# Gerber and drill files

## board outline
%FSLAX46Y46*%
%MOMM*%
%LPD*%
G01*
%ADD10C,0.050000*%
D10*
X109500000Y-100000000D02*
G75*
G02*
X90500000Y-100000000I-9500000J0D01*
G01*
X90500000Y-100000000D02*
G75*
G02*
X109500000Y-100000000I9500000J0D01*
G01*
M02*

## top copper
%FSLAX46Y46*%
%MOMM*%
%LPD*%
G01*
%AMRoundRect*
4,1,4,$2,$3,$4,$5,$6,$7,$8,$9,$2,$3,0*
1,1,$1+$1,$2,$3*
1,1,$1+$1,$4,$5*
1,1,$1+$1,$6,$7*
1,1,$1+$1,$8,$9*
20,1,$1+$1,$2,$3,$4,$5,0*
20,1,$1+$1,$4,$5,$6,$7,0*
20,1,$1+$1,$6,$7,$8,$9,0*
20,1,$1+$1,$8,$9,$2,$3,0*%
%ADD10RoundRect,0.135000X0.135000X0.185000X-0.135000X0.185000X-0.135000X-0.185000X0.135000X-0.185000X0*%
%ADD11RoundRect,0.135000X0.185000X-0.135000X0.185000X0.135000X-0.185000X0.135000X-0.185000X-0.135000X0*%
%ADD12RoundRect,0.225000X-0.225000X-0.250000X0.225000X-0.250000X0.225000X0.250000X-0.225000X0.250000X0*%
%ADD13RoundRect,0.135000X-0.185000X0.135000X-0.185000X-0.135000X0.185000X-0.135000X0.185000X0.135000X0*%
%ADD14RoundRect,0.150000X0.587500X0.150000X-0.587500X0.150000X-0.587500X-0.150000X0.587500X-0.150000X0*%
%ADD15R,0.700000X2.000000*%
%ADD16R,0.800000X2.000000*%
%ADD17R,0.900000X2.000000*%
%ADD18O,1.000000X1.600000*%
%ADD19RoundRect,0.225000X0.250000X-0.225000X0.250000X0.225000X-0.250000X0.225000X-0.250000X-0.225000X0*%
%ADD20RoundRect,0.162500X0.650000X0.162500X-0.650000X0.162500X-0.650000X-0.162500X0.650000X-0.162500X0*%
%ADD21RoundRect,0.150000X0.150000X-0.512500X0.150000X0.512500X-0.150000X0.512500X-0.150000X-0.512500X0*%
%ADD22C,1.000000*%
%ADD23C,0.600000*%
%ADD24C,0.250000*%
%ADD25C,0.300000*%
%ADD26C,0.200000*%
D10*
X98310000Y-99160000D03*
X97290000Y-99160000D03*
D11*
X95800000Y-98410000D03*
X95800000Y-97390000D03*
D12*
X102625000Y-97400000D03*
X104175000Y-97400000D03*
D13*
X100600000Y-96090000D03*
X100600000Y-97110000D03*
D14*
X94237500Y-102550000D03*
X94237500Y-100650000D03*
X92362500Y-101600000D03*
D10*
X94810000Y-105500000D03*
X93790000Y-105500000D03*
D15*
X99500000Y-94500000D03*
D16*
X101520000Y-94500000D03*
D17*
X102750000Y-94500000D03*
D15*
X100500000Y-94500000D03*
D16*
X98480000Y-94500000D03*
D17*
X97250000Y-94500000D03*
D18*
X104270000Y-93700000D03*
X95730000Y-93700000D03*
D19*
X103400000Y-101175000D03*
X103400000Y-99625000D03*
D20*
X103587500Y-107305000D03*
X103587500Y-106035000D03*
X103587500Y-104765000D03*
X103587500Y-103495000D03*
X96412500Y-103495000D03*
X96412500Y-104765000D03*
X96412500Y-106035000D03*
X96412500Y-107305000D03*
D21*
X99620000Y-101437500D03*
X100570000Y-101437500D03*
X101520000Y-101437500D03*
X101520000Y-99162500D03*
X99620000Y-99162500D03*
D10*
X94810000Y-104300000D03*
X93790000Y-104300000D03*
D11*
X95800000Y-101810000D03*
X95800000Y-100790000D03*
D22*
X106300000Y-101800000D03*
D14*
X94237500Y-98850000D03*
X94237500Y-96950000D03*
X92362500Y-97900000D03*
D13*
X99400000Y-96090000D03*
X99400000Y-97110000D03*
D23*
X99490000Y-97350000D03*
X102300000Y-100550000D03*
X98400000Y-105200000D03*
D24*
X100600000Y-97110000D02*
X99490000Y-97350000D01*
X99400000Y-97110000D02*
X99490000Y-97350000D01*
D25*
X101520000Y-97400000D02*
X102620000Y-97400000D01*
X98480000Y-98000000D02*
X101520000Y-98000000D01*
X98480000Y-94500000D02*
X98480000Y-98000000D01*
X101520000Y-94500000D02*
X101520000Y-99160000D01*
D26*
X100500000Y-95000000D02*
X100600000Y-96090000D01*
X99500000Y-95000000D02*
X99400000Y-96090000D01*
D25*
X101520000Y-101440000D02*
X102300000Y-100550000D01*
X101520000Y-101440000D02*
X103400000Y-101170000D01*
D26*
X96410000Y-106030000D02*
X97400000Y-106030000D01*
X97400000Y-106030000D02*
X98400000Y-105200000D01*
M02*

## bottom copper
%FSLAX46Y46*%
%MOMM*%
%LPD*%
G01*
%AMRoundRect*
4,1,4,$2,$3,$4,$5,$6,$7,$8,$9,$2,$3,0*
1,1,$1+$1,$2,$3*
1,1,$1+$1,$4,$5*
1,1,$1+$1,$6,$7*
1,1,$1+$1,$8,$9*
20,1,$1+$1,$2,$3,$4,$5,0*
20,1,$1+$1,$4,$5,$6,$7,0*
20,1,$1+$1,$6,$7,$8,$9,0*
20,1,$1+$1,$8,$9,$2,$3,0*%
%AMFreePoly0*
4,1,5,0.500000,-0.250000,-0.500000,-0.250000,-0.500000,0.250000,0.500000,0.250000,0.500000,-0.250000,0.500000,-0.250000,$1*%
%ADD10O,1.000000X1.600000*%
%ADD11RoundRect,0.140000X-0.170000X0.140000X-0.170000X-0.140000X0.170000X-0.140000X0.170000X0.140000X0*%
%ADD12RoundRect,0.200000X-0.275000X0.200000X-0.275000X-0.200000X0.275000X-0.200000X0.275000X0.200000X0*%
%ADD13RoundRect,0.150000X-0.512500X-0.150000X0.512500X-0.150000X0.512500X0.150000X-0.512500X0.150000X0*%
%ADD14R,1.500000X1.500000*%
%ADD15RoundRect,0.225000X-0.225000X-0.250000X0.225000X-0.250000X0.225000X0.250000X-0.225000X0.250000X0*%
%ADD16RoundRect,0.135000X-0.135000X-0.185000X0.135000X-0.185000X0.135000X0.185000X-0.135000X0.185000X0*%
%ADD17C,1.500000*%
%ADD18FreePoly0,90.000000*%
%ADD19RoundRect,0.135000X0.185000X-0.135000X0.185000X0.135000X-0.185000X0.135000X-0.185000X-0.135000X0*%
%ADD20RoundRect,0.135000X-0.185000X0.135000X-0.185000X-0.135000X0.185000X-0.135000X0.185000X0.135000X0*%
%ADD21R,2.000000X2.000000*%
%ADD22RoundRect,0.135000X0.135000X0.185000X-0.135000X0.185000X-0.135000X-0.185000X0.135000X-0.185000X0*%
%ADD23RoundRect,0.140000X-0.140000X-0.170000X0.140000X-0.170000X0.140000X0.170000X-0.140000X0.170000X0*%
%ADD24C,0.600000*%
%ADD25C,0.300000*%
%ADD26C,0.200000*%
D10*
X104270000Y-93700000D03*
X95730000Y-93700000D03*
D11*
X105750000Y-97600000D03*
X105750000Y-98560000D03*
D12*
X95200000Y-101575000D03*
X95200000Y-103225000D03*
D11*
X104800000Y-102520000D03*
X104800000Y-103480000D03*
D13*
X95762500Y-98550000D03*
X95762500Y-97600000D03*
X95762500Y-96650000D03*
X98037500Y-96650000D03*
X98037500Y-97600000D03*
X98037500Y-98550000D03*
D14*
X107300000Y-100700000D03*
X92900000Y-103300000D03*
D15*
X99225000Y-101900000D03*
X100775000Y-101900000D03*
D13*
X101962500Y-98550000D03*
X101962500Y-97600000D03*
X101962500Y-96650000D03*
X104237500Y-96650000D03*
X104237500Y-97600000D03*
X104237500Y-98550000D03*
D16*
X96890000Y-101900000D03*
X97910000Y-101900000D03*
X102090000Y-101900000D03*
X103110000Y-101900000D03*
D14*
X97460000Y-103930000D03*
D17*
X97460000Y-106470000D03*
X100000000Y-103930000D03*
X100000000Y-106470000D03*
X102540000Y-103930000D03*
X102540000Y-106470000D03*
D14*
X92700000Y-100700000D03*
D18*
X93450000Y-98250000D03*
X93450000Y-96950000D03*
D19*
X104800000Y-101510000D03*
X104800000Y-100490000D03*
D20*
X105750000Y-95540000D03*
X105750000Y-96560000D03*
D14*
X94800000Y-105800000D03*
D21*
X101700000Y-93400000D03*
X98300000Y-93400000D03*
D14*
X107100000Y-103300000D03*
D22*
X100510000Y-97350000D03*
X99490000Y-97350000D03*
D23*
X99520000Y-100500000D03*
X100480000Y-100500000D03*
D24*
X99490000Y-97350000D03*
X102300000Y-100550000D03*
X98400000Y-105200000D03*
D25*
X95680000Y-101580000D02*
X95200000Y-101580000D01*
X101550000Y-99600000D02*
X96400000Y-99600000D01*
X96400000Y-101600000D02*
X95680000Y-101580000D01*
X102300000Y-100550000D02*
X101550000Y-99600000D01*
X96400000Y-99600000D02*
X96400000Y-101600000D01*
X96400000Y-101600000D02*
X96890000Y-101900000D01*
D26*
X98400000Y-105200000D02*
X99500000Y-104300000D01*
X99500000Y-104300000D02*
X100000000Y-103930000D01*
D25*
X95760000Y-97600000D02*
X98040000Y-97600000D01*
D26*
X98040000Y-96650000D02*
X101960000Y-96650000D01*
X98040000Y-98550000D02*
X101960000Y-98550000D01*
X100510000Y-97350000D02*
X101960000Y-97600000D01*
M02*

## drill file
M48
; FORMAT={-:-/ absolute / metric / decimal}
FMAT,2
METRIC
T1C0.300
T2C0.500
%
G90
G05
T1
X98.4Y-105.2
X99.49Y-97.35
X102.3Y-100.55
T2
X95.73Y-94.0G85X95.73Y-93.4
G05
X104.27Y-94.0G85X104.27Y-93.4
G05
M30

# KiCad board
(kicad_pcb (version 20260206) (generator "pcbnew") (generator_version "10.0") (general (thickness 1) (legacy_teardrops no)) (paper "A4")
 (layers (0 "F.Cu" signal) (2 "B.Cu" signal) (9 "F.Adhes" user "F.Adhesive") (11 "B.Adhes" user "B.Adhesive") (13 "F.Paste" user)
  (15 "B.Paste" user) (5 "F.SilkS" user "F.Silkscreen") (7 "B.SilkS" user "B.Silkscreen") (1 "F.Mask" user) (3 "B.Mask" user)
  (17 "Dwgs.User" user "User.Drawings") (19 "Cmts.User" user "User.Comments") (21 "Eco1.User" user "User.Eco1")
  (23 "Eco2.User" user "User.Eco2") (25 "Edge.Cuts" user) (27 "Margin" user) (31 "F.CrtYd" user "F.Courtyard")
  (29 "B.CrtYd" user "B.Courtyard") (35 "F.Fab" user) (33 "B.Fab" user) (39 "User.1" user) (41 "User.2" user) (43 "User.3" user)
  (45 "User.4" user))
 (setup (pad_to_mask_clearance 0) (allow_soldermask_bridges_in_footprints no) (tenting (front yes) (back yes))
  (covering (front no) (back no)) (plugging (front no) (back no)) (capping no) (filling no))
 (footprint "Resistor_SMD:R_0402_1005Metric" (layer "F.Cu") (at 97.8 99.16 180)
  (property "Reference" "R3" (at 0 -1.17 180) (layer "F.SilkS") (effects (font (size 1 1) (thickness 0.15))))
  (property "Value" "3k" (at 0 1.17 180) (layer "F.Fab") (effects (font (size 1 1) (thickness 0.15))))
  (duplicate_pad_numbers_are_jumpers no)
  (pad "1" smd roundrect (at -0.51 0 180) (size 0.54 0.64) (layers "F.Cu" "F.Mask" "F.Paste") (roundrect_rratio 0.25) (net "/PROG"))
  (pad "2" smd roundrect (at 0.51 0 180) (size 0.54 0.64) (layers "F.Cu" "F.Mask" "F.Paste") (roundrect_rratio 0.25) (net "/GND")))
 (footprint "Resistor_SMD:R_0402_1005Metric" (layer "F.Cu") (at 95.8 97.9 90)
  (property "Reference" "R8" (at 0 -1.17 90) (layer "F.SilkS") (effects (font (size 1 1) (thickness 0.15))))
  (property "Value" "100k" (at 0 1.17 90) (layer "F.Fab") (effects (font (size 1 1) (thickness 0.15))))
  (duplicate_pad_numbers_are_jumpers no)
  (pad "1" smd roundrect (at -0.51 0 90) (size 0.54 0.64) (layers "F.Cu" "F.Mask" "F.Paste") (roundrect_rratio 0.25) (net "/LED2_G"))
  (pad "2" smd roundrect (at 0.51 0 90) (size 0.54 0.64) (layers "F.Cu" "F.Mask" "F.Paste") (roundrect_rratio 0.25) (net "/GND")))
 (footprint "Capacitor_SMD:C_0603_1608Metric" (layer "F.Cu") (at 103.4 97.4)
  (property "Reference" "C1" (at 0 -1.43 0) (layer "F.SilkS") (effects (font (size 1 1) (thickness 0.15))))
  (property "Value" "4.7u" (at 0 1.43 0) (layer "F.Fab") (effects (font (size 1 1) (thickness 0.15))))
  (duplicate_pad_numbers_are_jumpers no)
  (pad "1" smd roundrect (at -0.775 0) (size 0.9 0.95) (layers "F.Cu" "F.Mask" "F.Paste") (roundrect_rratio 0.25) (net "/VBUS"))
  (pad "2" smd roundrect (at 0.775 0) (size 0.9 0.95) (layers "F.Cu" "F.Mask" "F.Paste") (roundrect_rratio 0.25) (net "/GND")))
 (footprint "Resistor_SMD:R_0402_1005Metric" (layer "F.Cu") (at 100.6 96.6 -90)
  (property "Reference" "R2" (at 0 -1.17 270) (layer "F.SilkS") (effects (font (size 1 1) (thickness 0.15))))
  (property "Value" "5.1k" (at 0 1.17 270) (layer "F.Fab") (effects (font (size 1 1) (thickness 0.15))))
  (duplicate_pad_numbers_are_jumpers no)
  (pad "1" smd roundrect (at -0.51 0 270) (size 0.54 0.64) (layers "F.Cu" "F.Mask" "F.Paste") (roundrect_rratio 0.25) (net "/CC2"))
  (pad "2" smd roundrect (at 0.51 0 270) (size 0.54 0.64) (layers "F.Cu" "F.Mask" "F.Paste") (roundrect_rratio 0.25) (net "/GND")))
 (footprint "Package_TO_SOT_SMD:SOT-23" (layer "F.Cu") (at 93.3 101.6 180)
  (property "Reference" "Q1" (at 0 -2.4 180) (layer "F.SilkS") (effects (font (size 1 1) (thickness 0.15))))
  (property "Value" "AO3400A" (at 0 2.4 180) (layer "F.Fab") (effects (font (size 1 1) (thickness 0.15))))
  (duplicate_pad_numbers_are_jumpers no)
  (pad "1" smd roundrect (at -0.9375 -0.95 180) (size 1.475 0.6) (layers "F.Cu" "F.Mask" "F.Paste") (roundrect_rratio 0.25) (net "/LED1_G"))
  (pad "2" smd roundrect (at -0.9375 0.95 180) (size 1.475 0.6) (layers "F.Cu" "F.Mask" "F.Paste") (roundrect_rratio 0.25) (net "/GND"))
  (pad "3" smd roundrect (at 0.9375 0 180) (size 1.475 0.6) (layers "F.Cu" "F.Mask" "F.Paste") (roundrect_rratio 0.25) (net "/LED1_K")))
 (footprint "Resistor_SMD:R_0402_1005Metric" (layer "F.Cu") (at 94.3 105.5 180)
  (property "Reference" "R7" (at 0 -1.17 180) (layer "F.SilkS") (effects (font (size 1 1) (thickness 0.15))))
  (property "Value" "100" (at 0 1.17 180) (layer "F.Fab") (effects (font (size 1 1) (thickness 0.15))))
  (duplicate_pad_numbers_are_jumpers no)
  (pad "1" smd roundrect (at -0.51 0 180) (size 0.54 0.64) (layers "F.Cu" "F.Mask" "F.Paste") (roundrect_rratio 0.25) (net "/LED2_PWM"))
  (pad "2" smd roundrect (at 0.51 0 180) (size 0.54 0.64) (layers "F.Cu" "F.Mask" "F.Paste") (roundrect_rratio 0.25) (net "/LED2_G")))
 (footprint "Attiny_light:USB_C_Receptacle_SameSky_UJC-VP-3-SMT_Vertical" (layer "F.Cu") (at 100 94.5 180)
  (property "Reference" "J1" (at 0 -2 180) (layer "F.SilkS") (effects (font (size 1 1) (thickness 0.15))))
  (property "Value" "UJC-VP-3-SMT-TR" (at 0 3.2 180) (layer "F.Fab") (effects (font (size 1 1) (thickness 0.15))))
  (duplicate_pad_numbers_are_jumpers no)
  (pad "A5" smd rect (at 0.5 0 180) (size 0.7 2) (layers "F.Cu" "F.Mask" "F.Paste") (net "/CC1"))
  (pad "A9" smd rect (at -1.52 0 180) (size 0.8 2) (layers "F.Cu" "F.Mask" "F.Paste") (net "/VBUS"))
  (pad "A12" smd rect (at -2.75 0 180) (size 0.9 2) (layers "F.Cu" "F.Mask" "F.Paste") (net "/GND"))
  (pad "B5" smd rect (at -0.5 0 180) (size 0.7 2) (layers "F.Cu" "F.Mask" "F.Paste") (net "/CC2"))
  (pad "B9" smd rect (at 1.52 0 180) (size 0.8 2) (layers "F.Cu" "F.Mask" "F.Paste") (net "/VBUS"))
  (pad "B12" smd rect (at 2.75 0 180) (size 0.9 2) (layers "F.Cu" "F.Mask" "F.Paste") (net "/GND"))
  (pad "SH" thru_hole oval (at -4.27 0.8 180) (size 1 1.6) (drill oval 0.5 1.1) (layers "*.Cu" "*.Mask") (remove_unused_layers no)
   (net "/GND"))
  (pad "SH" thru_hole oval (at 4.27 0.8 180) (size 1 1.6) (drill oval 0.5 1.1) (layers "*.Cu" "*.Mask") (remove_unused_layers no)
   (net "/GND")))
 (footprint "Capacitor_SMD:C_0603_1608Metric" (layer "F.Cu") (at 103.4 100.4 90)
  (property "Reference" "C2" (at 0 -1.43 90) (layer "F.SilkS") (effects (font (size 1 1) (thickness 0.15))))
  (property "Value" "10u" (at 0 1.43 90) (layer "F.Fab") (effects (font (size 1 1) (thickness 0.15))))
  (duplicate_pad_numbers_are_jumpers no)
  (pad "1" smd roundrect (at -0.775 0 90) (size 0.9 0.95) (layers "F.Cu" "F.Mask" "F.Paste") (roundrect_rratio 0.25) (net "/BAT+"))
  (pad "2" smd roundrect (at 0.775 0 90) (size 0.9 0.95) (layers "F.Cu" "F.Mask" "F.Paste") (roundrect_rratio 0.25) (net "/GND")))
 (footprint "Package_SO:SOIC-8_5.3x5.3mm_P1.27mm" (layer "F.Cu") (at 100 105.4 180)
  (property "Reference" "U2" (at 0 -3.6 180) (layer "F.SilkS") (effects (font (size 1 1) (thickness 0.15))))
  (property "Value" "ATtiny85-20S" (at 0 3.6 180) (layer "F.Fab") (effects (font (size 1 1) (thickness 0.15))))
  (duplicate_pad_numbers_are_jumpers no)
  (pad "1" smd roundrect (at -3.5875 -1.905 180) (size 1.625 0.65) (layers "F.Cu" "F.Mask" "F.Paste") (roundrect_rratio 0.25) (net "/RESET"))
  (pad "2" smd roundrect (at -3.5875 -0.635 180) (size 1.625 0.65) (layers "F.Cu" "F.Mask" "F.Paste") (roundrect_rratio 0.25) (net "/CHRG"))
  (pad "3" smd roundrect (at -3.5875 0.635 180) (size 1.625 0.65) (layers "F.Cu" "F.Mask" "F.Paste") (roundrect_rratio 0.25) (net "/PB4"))
  (pad "4" smd roundrect (at -3.5875 1.905 180) (size 1.625 0.65) (layers "F.Cu" "F.Mask" "F.Paste") (roundrect_rratio 0.25) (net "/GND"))
  (pad "5" smd roundrect (at 3.5875 1.905 180) (size 1.625 0.65) (layers "F.Cu" "F.Mask" "F.Paste") (roundrect_rratio 0.25)
   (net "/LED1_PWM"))
  (pad "6" smd roundrect (at 3.5875 0.635 180) (size 1.625 0.65) (layers "F.Cu" "F.Mask" "F.Paste") (roundrect_rratio 0.25)
   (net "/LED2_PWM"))
  (pad "7" smd roundrect (at 3.5875 -0.635 180) (size 1.625 0.65) (layers "F.Cu" "F.Mask" "F.Paste") (roundrect_rratio 0.25) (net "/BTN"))
  (pad "8" smd roundrect (at 3.5875 -1.905 180) (size 1.625 0.65) (layers "F.Cu" "F.Mask" "F.Paste") (roundrect_rratio 0.25) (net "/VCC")))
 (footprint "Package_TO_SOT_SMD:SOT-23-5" (layer "F.Cu") (at 100.57 100.3 90)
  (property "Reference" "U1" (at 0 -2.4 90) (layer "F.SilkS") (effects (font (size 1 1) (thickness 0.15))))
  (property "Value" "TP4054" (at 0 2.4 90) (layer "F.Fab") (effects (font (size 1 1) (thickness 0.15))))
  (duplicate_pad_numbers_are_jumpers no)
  (pad "1" smd roundrect (at -1.1375 -0.95 90) (size 1.325 0.6) (layers "F.Cu" "F.Mask" "F.Paste") (roundrect_rratio 0.25) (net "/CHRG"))
  (pad "2" smd roundrect (at -1.1375 0 90) (size 1.325 0.6) (layers "F.Cu" "F.Mask" "F.Paste") (roundrect_rratio 0.25) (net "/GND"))
  (pad "3" smd roundrect (at -1.1375 0.95 90) (size 1.325 0.6) (layers "F.Cu" "F.Mask" "F.Paste") (roundrect_rratio 0.25) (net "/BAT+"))
  (pad "4" smd roundrect (at 1.1375 0.95 90) (size 1.325 0.6) (layers "F.Cu" "F.Mask" "F.Paste") (roundrect_rratio 0.25) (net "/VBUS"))
  (pad "5" smd roundrect (at 1.1375 -0.95 90) (size 1.325 0.6) (layers "F.Cu" "F.Mask" "F.Paste") (roundrect_rratio 0.25) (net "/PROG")))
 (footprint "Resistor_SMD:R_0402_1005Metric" (layer "F.Cu") (at 94.3 104.3 180)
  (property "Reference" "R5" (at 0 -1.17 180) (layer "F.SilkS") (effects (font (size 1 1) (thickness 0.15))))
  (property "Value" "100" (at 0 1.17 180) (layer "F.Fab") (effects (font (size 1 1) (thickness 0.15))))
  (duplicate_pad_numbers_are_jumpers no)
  (pad "1" smd roundrect (at -0.51 0 180) (size 0.54 0.64) (layers "F.Cu" "F.Mask" "F.Paste") (roundrect_rratio 0.25) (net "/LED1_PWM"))
  (pad "2" smd roundrect (at 0.51 0 180) (size 0.54 0.64) (layers "F.Cu" "F.Mask" "F.Paste") (roundrect_rratio 0.25) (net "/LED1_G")))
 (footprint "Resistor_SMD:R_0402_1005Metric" (layer "F.Cu") (at 95.8 101.3 90)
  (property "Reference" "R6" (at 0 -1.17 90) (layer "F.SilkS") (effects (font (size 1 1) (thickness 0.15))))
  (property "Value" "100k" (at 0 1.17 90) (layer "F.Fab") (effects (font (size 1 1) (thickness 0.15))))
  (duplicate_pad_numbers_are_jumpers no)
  (pad "1" smd roundrect (at -0.51 0 90) (size 0.54 0.64) (layers "F.Cu" "F.Mask" "F.Paste") (roundrect_rratio 0.25) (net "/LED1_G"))
  (pad "2" smd roundrect (at 0.51 0 90) (size 0.54 0.64) (layers "F.Cu" "F.Mask" "F.Paste") (roundrect_rratio 0.25) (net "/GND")))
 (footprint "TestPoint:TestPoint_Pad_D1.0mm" (layer "F.Cu") (at 106.3 101.8)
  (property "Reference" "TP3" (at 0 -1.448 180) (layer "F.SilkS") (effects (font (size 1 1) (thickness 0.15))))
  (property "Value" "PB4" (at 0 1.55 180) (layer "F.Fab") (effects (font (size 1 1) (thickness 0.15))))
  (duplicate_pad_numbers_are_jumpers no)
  (pad "1" smd circle (at 0 0) (size 1 1) (layers "F.Cu" "F.Mask") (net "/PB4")))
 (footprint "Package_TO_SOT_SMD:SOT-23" (layer "F.Cu") (at 93.3 97.9 180)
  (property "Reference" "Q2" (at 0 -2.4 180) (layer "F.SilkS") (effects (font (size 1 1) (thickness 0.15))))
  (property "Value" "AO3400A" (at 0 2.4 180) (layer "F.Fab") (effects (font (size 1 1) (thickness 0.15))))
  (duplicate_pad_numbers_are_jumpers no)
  (pad "1" smd roundrect (at -0.9375 -0.95 180) (size 1.475 0.6) (layers "F.Cu" "F.Mask" "F.Paste") (roundrect_rratio 0.25) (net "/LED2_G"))
  (pad "2" smd roundrect (at -0.9375 0.95 180) (size 1.475 0.6) (layers "F.Cu" "F.Mask" "F.Paste") (roundrect_rratio 0.25) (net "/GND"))
  (pad "3" smd roundrect (at 0.9375 0 180) (size 1.475 0.6) (layers "F.Cu" "F.Mask" "F.Paste") (roundrect_rratio 0.25) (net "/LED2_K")))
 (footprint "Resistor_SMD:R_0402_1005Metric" (layer "F.Cu") (at 99.4 96.6 -90)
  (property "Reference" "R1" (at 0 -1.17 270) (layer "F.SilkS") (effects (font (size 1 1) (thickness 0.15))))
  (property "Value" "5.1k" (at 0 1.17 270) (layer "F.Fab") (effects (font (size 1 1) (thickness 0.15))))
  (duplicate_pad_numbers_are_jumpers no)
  (pad "1" smd roundrect (at -0.51 0 270) (size 0.54 0.64) (layers "F.Cu" "F.Mask" "F.Paste") (roundrect_rratio 0.25) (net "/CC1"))
  (pad "2" smd roundrect (at 0.51 0 270) (size 0.54 0.64) (layers "F.Cu" "F.Mask" "F.Paste") (roundrect_rratio 0.25) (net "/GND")))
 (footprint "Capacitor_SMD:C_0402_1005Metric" (layer "B.Cu") (at 105.75 98.08 -90)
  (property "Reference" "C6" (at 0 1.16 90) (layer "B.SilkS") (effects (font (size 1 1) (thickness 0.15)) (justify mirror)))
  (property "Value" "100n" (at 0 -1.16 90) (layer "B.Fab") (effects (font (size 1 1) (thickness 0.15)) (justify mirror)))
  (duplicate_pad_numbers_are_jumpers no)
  (pad "1" smd roundrect (at -0.48 0 270) (size 0.56 0.62) (layers "B.Cu" "B.Mask" "B.Paste") (roundrect_rratio 0.25) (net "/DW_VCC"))
  (pad "2" smd roundrect (at 0.48 0 270) (size 0.56 0.62) (layers "B.Cu" "B.Mask" "B.Paste") (roundrect_rratio 0.25) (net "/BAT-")))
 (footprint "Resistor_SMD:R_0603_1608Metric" (layer "B.Cu") (at 95.2 102.4 -90)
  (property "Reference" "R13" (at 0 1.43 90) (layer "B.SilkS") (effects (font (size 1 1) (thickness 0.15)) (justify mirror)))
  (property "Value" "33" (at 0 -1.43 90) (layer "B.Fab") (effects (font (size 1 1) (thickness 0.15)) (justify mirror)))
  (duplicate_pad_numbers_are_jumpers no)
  (pad "1" smd roundrect (at -0.825 0 270) (size 0.8 0.95) (layers "B.Cu" "B.Mask" "B.Paste") (roundrect_rratio 0.25) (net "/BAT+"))
  (pad "2" smd roundrect (at 0.825 0 270) (size 0.8 0.95) (layers "B.Cu" "B.Mask" "B.Paste") (roundrect_rratio 0.25) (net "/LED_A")))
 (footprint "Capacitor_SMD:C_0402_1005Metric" (layer "B.Cu") (at 104.8 103 -90)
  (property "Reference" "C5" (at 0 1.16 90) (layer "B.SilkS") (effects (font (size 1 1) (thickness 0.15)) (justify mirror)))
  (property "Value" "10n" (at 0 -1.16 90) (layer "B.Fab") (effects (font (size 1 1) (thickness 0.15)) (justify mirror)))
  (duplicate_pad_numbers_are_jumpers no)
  (pad "1" smd roundrect (at -0.48 0 270) (size 0.56 0.62) (layers "B.Cu" "B.Mask" "B.Paste") (roundrect_rratio 0.25) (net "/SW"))
  (pad "2" smd roundrect (at 0.48 0 270) (size 0.56 0.62) (layers "B.Cu" "B.Mask" "B.Paste") (roundrect_rratio 0.25) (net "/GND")))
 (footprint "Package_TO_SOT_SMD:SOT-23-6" (layer "B.Cu") (at 96.9 97.6)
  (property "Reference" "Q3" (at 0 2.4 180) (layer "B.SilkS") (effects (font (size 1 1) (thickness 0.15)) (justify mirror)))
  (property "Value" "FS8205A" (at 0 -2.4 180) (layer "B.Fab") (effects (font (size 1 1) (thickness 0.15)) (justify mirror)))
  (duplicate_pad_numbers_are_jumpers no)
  (pad "1" smd roundrect (at -1.1375 0.95) (size 1.325 0.6) (layers "B.Cu" "B.Mask" "B.Paste") (roundrect_rratio 0.25) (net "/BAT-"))
  (pad "2" smd roundrect (at -1.1375 0) (size 1.325 0.6) (layers "B.Cu" "B.Mask" "B.Paste") (roundrect_rratio 0.25) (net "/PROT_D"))
  (pad "3" smd roundrect (at -1.1375 -0.95) (size 1.325 0.6) (layers "B.Cu" "B.Mask" "B.Paste") (roundrect_rratio 0.25) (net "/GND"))
  (pad "4" smd roundrect (at 1.1375 -0.95) (size 1.325 0.6) (layers "B.Cu" "B.Mask" "B.Paste") (roundrect_rratio 0.25) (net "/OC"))
  (pad "5" smd roundrect (at 1.1375 0) (size 1.325 0.6) (layers "B.Cu" "B.Mask" "B.Paste") (roundrect_rratio 0.25) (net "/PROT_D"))
  (pad "6" smd roundrect (at 1.1375 0.95) (size 1.325 0.6) (layers "B.Cu" "B.Mask" "B.Paste") (roundrect_rratio 0.25) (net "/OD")))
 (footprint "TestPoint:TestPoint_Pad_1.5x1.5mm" (layer "B.Cu") (at 107.3 100.7)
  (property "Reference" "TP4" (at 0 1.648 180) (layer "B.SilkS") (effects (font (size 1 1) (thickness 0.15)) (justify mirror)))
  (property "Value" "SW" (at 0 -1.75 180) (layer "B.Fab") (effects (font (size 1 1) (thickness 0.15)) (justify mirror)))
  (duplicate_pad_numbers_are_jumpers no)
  (pad "1" smd rect (at 0 0) (size 1.5 1.5) (layers "B.Cu" "B.Mask") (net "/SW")))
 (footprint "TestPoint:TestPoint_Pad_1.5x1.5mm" (layer "B.Cu") (at 92.9 103.3)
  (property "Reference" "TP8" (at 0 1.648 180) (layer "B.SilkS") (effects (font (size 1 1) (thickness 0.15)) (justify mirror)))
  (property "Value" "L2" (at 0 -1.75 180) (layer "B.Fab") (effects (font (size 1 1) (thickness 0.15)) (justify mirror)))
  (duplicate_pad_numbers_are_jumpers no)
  (pad "1" smd rect (at 0 0) (size 1.5 1.5) (layers "B.Cu" "B.Mask") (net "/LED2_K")))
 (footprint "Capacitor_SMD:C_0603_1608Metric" (layer "B.Cu") (at 100 101.9)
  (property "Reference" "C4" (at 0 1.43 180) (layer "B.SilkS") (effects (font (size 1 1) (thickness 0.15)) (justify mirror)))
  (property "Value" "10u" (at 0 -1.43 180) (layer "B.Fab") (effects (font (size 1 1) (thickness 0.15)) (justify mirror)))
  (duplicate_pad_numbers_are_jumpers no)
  (pad "1" smd roundrect (at -0.775 0) (size 0.9 0.95) (layers "B.Cu" "B.Mask" "B.Paste") (roundrect_rratio 0.25) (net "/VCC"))
  (pad "2" smd roundrect (at 0.775 0) (size 0.9 0.95) (layers "B.Cu" "B.Mask" "B.Paste") (roundrect_rratio 0.25) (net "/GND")))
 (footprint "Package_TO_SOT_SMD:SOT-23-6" (layer "B.Cu") (at 103.1 97.6)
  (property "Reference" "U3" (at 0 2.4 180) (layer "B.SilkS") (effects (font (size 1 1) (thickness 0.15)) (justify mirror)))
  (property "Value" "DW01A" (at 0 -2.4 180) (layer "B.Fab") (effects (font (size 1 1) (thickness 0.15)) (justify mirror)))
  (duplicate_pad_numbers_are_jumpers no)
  (pad "1" smd roundrect (at -1.1375 0.95) (size 1.325 0.6) (layers "B.Cu" "B.Mask" "B.Paste") (roundrect_rratio 0.25) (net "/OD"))
  (pad "2" smd roundrect (at -1.1375 0) (size 1.325 0.6) (layers "B.Cu" "B.Mask" "B.Paste") (roundrect_rratio 0.25) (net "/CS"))
  (pad "3" smd roundrect (at -1.1375 -0.95) (size 1.325 0.6) (layers "B.Cu" "B.Mask" "B.Paste") (roundrect_rratio 0.25) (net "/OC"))
  (pad "4" smd roundrect (at 1.1375 -0.95) (size 1.325 0.6) (layers "B.Cu" "B.Mask" "B.Paste") (roundrect_rratio 0.25)
   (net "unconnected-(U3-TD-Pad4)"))
  (pad "5" smd roundrect (at 1.1375 0) (size 1.325 0.6) (layers "B.Cu" "B.Mask" "B.Paste") (roundrect_rratio 0.25) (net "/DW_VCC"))
  (pad "6" smd roundrect (at 1.1375 0.95) (size 1.325 0.6) (layers "B.Cu" "B.Mask" "B.Paste") (roundrect_rratio 0.25) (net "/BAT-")))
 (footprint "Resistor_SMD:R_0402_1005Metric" (layer "B.Cu") (at 97.4 101.9)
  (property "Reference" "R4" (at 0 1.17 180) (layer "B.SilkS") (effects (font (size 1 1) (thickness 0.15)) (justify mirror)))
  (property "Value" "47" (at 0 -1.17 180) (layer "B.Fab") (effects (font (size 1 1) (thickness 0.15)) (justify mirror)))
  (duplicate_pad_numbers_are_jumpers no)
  (pad "1" smd roundrect (at -0.51 0) (size 0.54 0.64) (layers "B.Cu" "B.Mask" "B.Paste") (roundrect_rratio 0.25) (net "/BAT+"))
  (pad "2" smd roundrect (at 0.51 0) (size 0.54 0.64) (layers "B.Cu" "B.Mask" "B.Paste") (roundrect_rratio 0.25) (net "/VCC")))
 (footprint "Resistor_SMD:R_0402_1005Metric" (layer "B.Cu") (at 102.6 101.9)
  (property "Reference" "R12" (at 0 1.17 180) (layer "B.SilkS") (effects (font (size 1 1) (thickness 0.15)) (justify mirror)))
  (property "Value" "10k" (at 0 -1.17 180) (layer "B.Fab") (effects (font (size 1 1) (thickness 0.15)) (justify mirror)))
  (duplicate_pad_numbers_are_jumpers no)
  (pad "1" smd roundrect (at -0.51 0) (size 0.54 0.64) (layers "B.Cu" "B.Mask" "B.Paste") (roundrect_rratio 0.25) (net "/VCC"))
  (pad "2" smd roundrect (at 0.51 0) (size 0.54 0.64) (layers "B.Cu" "B.Mask" "B.Paste") (roundrect_rratio 0.25) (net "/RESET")))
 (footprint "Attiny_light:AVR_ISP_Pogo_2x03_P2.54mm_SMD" (layer "B.Cu") (at 100 105.2 -90)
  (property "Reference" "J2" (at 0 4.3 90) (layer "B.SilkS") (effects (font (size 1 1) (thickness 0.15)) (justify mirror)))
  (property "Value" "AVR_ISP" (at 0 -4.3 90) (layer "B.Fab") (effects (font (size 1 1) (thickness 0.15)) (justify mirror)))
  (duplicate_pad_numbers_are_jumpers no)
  (pad "1" smd rect (at -1.27 2.54 270) (size 1.5 1.5) (layers "B.Cu" "B.Mask" "B.Paste") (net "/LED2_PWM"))
  (pad "2" smd circle (at 1.27 2.54 270) (size 1.5 1.5) (layers "B.Cu" "B.Mask" "B.Paste") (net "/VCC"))
  (pad "3" smd circle (at -1.27 0 270) (size 1.5 1.5) (layers "B.Cu" "B.Mask" "B.Paste") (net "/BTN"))
  (pad "4" smd circle (at 1.27 0 270) (size 1.5 1.5) (layers "B.Cu" "B.Mask" "B.Paste") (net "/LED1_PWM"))
  (pad "5" smd circle (at -1.27 -2.54 270) (size 1.5 1.5) (layers "B.Cu" "B.Mask" "B.Paste") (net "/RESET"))
  (pad "6" smd circle (at 1.27 -2.54 270) (size 1.5 1.5) (layers "B.Cu" "B.Mask" "B.Paste") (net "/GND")))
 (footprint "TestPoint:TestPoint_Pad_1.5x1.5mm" (layer "B.Cu") (at 92.7 100.7)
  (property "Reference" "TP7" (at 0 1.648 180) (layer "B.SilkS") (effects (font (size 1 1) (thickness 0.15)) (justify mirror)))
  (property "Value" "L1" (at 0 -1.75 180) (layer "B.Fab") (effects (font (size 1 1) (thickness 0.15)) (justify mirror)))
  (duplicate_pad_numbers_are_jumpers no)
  (pad "1" smd rect (at 0 0) (size 1.5 1.5) (layers "B.Cu" "B.Mask") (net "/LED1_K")))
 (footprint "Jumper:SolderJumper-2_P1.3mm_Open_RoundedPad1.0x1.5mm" (layer "B.Cu") (at 93.45 97.6 90)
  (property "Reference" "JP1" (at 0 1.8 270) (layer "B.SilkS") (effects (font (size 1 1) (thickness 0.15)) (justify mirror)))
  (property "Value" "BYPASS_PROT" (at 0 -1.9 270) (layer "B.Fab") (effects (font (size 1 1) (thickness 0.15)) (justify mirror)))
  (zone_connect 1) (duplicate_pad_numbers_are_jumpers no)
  (pad "1" smd custom (at -0.65 0 90) (size 1 0.5) (layers "B.Cu" "B.Mask") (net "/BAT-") (zone_connect 2) (thermal_bridge_angle 45)
   (options (clearance outline) (anchor rect)) (primitives))
  (pad "2" smd custom (at 0.65 0 90) (size 1 0.5) (layers "B.Cu" "B.Mask") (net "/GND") (zone_connect 2) (thermal_bridge_angle 45)
   (options (clearance outline) (anchor rect)) (primitives)))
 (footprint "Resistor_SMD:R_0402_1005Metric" (layer "B.Cu") (at 104.8 101 90)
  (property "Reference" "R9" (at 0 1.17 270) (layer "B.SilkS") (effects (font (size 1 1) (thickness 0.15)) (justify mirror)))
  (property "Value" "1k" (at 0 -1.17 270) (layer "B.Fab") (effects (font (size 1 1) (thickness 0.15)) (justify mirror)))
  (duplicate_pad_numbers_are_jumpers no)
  (pad "1" smd roundrect (at -0.51 0 90) (size 0.54 0.64) (layers "B.Cu" "B.Mask" "B.Paste") (roundrect_rratio 0.25) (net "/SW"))
  (pad "2" smd roundrect (at 0.51 0 90) (size 0.54 0.64) (layers "B.Cu" "B.Mask" "B.Paste") (roundrect_rratio 0.25) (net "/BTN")))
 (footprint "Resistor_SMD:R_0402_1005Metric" (layer "B.Cu") (at 105.75 96.05 -90)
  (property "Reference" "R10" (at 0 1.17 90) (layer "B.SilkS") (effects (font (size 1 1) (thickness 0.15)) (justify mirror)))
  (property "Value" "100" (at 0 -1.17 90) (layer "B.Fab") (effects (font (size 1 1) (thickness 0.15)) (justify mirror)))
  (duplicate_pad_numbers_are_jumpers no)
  (pad "1" smd roundrect (at -0.51 0 270) (size 0.54 0.64) (layers "B.Cu" "B.Mask" "B.Paste") (roundrect_rratio 0.25) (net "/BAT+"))
  (pad "2" smd roundrect (at 0.51 0 270) (size 0.54 0.64) (layers "B.Cu" "B.Mask" "B.Paste") (roundrect_rratio 0.25) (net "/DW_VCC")))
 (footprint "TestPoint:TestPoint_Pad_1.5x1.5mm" (layer "B.Cu") (at 94.8 105.8)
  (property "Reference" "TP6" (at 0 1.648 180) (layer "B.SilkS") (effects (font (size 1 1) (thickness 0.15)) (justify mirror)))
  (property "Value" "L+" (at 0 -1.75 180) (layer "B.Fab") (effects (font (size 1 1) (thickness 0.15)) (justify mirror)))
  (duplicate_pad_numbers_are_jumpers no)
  (pad "1" smd rect (at 0 0) (size 1.5 1.5) (layers "B.Cu" "B.Mask") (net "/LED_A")))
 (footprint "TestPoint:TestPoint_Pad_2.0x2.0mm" (layer "B.Cu") (at 101.7 93.4)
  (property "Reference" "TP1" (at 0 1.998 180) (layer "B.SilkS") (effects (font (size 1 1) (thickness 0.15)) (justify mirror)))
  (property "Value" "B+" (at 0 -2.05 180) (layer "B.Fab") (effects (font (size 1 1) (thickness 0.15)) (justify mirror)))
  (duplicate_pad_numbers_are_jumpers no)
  (pad "1" smd rect (at 0 0) (size 2 2) (layers "B.Cu" "B.Mask") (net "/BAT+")))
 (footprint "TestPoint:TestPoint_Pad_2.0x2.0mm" (layer "B.Cu") (at 98.3 93.4)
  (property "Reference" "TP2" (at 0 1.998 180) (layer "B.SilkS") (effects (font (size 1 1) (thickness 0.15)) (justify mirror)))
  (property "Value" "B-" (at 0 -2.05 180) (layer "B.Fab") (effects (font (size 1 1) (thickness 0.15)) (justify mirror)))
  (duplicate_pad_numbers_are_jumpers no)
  (pad "1" smd rect (at 0 0) (size 2 2) (layers "B.Cu" "B.Mask") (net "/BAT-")))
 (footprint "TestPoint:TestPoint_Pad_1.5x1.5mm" (layer "B.Cu") (at 107.1 103.3)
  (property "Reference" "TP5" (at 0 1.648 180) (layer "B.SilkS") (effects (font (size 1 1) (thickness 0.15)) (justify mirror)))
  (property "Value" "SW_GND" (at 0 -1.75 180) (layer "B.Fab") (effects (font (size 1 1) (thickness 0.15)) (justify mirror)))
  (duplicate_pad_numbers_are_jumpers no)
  (pad "1" smd rect (at 0 0) (size 1.5 1.5) (layers "B.Cu" "B.Mask") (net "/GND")))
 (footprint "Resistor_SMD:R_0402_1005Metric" (layer "B.Cu") (at 100 97.35 180)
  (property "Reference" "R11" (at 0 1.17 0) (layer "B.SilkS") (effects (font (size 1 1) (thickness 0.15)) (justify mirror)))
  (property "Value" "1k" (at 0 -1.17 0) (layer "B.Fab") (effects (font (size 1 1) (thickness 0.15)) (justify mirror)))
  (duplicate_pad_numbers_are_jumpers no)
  (pad "1" smd roundrect (at -0.51 0 180) (size 0.54 0.64) (layers "B.Cu" "B.Mask" "B.Paste") (roundrect_rratio 0.25) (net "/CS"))
  (pad "2" smd roundrect (at 0.51 0 180) (size 0.54 0.64) (layers "B.Cu" "B.Mask" "B.Paste") (roundrect_rratio 0.25) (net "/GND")))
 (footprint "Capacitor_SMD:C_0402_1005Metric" (layer "B.Cu") (at 100 100.5)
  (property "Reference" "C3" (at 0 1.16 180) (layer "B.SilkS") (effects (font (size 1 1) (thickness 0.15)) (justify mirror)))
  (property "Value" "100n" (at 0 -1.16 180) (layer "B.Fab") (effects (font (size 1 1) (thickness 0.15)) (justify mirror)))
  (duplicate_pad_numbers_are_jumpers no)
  (pad "1" smd roundrect (at -0.48 0) (size 0.56 0.62) (layers "B.Cu" "B.Mask" "B.Paste") (roundrect_rratio 0.25) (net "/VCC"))
  (pad "2" smd roundrect (at 0.48 0) (size 0.56 0.62) (layers "B.Cu" "B.Mask" "B.Paste") (roundrect_rratio 0.25) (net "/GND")))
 (gr_circle (center 100 100) (end 109.5 100) (stroke (width 0.05) (type default)) (fill no) (layer "Edge.Cuts"))
 (segment (start 100.6 97.11) (end 99.49 97.35) (width 0.25) (locked yes) (layer "F.Cu") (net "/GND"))
 (segment (start 99.4 97.11) (end 99.49 97.35) (width 0.25) (locked yes) (layer "F.Cu") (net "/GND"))
 (via (at 99.49 97.35) (size 0.6) (drill 0.3) (layers "F.Cu" "B.Cu") (locked yes) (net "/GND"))
 (segment (start 101.52 97.4) (end 102.62 97.4) (width 0.3) (locked yes) (layer "F.Cu") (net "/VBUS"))
 (segment (start 98.48 98) (end 101.52 98) (width 0.3) (locked yes) (layer "F.Cu") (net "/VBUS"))
 (segment (start 98.48 94.5) (end 98.48 98) (width 0.3) (locked yes) (layer "F.Cu") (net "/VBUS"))
 (segment (start 101.52 94.5) (end 101.52 99.16) (width 0.3) (locked yes) (layer "F.Cu") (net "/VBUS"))
 (segment (start 100.5 95) (end 100.6 96.09) (width 0.2) (locked yes) (layer "F.Cu") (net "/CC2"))
 (segment (start 99.5 95) (end 99.4 96.09) (width 0.2) (locked yes) (layer "F.Cu") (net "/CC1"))
 (segment (start 101.52 101.44) (end 102.3 100.55) (width 0.3) (locked yes) (layer "F.Cu") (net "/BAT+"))
 (segment (start 101.52 101.44) (end 103.4 101.17) (width 0.3) (locked yes) (layer "F.Cu") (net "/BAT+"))
 (via (at 102.3 100.55) (size 0.6) (drill 0.3) (layers "F.Cu" "B.Cu") (locked yes) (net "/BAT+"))
 (segment (start 95.68 101.58) (end 95.2 101.58) (width 0.3) (locked yes) (layer "B.Cu") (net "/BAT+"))
 (segment (start 101.55 99.6) (end 96.4 99.6) (width 0.3) (locked yes) (layer "B.Cu") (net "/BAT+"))
 (segment (start 96.4 101.6) (end 95.68 101.58) (width 0.3) (locked yes) (layer "B.Cu") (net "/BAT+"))
 (segment (start 102.3 100.55) (end 101.55 99.6) (width 0.3) (locked yes) (layer "B.Cu") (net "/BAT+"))
 (segment (start 96.4 99.6) (end 96.4 101.6) (width 0.3) (locked yes) (layer "B.Cu") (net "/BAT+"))
 (segment (start 96.4 101.6) (end 96.89 101.9) (width 0.3) (locked yes) (layer "B.Cu") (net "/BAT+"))
 (segment (start 96.41 106.03) (end 97.4 106.03) (width 0.2) (locked yes) (layer "F.Cu") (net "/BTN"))
 (segment (start 97.4 106.03) (end 98.4 105.2) (width 0.2) (locked yes) (layer "F.Cu") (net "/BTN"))
 (via (at 98.4 105.2) (size 0.6) (drill 0.3) (layers "F.Cu" "B.Cu") (locked yes) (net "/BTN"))
 (segment (start 98.4 105.2) (end 99.5 104.3) (width 0.2) (locked yes) (layer "B.Cu") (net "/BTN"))
 (segment (start 99.5 104.3) (end 100 103.93) (width 0.2) (locked yes) (layer "B.Cu") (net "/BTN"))
 (segment (start 95.76 97.6) (end 98.04 97.6) (width 0.3) (locked yes) (layer "B.Cu") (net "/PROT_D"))
 (segment (start 98.04 96.65) (end 101.96 96.65) (width 0.2) (locked yes) (layer "B.Cu") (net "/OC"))
 (segment (start 98.04 98.55) (end 101.96 98.55) (width 0.2) (locked yes) (layer "B.Cu") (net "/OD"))
 (segment (start 100.51 97.35) (end 101.96 97.6) (width 0.2) (locked yes) (layer "B.Cu") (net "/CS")))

